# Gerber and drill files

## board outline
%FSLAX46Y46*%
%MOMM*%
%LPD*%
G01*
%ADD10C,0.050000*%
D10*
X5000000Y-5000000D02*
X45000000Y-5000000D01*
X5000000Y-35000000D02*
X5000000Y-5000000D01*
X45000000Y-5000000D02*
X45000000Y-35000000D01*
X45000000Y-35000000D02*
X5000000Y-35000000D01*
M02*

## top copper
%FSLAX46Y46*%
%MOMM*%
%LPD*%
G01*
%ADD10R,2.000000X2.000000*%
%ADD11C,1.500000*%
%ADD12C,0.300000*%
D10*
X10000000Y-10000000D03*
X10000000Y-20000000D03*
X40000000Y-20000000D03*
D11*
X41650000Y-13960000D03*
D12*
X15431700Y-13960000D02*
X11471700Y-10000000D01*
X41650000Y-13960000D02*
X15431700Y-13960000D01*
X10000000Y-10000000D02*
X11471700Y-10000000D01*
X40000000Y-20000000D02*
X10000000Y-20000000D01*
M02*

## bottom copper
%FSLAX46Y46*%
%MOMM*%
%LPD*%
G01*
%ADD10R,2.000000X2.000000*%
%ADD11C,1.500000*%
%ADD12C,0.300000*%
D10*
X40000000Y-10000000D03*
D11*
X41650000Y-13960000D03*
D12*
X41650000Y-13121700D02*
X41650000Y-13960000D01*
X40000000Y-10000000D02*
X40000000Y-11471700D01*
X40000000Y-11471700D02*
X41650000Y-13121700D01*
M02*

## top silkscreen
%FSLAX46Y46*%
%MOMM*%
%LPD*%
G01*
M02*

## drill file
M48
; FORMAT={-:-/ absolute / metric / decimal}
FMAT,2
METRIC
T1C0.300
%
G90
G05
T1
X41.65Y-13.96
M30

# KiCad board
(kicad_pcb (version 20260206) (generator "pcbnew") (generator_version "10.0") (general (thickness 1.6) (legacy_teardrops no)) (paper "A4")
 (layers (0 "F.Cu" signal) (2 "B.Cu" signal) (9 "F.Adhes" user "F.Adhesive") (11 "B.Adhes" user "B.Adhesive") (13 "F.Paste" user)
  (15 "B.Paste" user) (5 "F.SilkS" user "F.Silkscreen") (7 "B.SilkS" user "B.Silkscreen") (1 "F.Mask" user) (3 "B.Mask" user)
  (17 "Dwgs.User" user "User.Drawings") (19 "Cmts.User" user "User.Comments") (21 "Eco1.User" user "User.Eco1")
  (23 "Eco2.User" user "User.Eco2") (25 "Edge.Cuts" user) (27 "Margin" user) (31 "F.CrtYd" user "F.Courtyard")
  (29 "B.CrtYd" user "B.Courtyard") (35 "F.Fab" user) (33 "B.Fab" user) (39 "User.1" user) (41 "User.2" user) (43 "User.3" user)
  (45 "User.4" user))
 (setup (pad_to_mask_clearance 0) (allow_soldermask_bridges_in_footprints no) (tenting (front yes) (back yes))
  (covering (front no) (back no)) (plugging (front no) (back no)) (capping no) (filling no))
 (gr_line (start 5 5) (end 45 5) (stroke (width 0.05) (type default)) (layer "Edge.Cuts"))
 (gr_line (start 5 35) (end 5 5) (stroke (width 0.05) (type default)) (layer "Edge.Cuts"))
 (gr_line (start 45 5) (end 45 35) (stroke (width 0.05) (type default)) (layer "Edge.Cuts"))
 (gr_line (start 45 35) (end 5 35) (stroke (width 0.05) (type default)) (layer "Edge.Cuts"))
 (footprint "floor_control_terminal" (layer "F.Cu") (at 10 10)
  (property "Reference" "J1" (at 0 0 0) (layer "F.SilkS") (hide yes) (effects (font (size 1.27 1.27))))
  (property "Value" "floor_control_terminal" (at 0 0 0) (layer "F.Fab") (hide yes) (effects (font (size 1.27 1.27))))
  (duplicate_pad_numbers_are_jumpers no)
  (pad "1" smd rect (at 0 0) (size 2 2) (layers "F.Cu" "F.Paste" "F.Mask") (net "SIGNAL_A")))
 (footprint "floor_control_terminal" (layer "B.Cu") (at 40 10)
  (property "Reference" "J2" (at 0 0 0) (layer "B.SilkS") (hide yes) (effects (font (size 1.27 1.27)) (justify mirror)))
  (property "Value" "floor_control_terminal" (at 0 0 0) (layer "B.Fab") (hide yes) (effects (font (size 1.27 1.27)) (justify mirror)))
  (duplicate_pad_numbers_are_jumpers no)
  (pad "1" smd rect (at 0 0) (size 2 2) (layers "B.Cu" "B.Paste" "B.Mask") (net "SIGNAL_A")))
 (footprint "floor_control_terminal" (layer "F.Cu") (at 10 20)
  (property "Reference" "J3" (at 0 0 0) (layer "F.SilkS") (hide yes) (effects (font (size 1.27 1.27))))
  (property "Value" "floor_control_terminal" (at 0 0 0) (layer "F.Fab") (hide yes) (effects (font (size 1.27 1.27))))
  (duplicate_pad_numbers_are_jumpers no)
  (pad "1" smd rect (at 0 0) (size 2 2) (layers "F.Cu" "F.Paste" "F.Mask") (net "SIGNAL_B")))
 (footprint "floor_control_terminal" (layer "F.Cu") (at 40 20)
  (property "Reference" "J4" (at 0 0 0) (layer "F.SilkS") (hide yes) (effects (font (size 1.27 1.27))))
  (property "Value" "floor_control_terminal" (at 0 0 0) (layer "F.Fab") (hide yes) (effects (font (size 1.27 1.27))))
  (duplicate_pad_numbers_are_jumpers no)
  (pad "1" smd rect (at 0 0) (size 2 2) (layers "F.Cu" "F.Paste" "F.Mask") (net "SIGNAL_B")))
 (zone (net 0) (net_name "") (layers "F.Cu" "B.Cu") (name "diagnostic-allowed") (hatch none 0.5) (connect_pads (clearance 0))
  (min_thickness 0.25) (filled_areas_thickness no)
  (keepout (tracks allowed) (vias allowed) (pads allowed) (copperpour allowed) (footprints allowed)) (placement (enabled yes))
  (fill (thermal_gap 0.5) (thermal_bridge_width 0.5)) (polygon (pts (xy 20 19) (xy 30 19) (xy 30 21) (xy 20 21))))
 (segment (start 15.4317 13.96) (end 11.4717 10) (width 0.3) (layer "F.Cu") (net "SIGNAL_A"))
 (segment (start 41.65 13.96) (end 15.4317 13.96) (width 0.3) (layer "F.Cu") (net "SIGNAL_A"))
 (segment (start 10 10) (end 11.4717 10) (width 0.3) (layer "F.Cu") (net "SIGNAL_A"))
 (via (at 41.65 13.96) (size 1.5) (drill 0.3) (layers "F.Cu" "B.Cu") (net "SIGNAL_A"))
 (segment (start 41.65 13.1217) (end 41.65 13.96) (width 0.3) (layer "B.Cu") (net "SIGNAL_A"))
 (segment (start 40 10) (end 40 11.4717) (width 0.3) (layer "B.Cu") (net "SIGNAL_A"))
 (segment (start 40 11.4717) (end 41.65 13.1217) (width 0.3) (layer "B.Cu") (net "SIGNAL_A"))
 (segment (start 40 20) (end 10 20) (width 0.3) (layer "F.Cu") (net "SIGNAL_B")))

